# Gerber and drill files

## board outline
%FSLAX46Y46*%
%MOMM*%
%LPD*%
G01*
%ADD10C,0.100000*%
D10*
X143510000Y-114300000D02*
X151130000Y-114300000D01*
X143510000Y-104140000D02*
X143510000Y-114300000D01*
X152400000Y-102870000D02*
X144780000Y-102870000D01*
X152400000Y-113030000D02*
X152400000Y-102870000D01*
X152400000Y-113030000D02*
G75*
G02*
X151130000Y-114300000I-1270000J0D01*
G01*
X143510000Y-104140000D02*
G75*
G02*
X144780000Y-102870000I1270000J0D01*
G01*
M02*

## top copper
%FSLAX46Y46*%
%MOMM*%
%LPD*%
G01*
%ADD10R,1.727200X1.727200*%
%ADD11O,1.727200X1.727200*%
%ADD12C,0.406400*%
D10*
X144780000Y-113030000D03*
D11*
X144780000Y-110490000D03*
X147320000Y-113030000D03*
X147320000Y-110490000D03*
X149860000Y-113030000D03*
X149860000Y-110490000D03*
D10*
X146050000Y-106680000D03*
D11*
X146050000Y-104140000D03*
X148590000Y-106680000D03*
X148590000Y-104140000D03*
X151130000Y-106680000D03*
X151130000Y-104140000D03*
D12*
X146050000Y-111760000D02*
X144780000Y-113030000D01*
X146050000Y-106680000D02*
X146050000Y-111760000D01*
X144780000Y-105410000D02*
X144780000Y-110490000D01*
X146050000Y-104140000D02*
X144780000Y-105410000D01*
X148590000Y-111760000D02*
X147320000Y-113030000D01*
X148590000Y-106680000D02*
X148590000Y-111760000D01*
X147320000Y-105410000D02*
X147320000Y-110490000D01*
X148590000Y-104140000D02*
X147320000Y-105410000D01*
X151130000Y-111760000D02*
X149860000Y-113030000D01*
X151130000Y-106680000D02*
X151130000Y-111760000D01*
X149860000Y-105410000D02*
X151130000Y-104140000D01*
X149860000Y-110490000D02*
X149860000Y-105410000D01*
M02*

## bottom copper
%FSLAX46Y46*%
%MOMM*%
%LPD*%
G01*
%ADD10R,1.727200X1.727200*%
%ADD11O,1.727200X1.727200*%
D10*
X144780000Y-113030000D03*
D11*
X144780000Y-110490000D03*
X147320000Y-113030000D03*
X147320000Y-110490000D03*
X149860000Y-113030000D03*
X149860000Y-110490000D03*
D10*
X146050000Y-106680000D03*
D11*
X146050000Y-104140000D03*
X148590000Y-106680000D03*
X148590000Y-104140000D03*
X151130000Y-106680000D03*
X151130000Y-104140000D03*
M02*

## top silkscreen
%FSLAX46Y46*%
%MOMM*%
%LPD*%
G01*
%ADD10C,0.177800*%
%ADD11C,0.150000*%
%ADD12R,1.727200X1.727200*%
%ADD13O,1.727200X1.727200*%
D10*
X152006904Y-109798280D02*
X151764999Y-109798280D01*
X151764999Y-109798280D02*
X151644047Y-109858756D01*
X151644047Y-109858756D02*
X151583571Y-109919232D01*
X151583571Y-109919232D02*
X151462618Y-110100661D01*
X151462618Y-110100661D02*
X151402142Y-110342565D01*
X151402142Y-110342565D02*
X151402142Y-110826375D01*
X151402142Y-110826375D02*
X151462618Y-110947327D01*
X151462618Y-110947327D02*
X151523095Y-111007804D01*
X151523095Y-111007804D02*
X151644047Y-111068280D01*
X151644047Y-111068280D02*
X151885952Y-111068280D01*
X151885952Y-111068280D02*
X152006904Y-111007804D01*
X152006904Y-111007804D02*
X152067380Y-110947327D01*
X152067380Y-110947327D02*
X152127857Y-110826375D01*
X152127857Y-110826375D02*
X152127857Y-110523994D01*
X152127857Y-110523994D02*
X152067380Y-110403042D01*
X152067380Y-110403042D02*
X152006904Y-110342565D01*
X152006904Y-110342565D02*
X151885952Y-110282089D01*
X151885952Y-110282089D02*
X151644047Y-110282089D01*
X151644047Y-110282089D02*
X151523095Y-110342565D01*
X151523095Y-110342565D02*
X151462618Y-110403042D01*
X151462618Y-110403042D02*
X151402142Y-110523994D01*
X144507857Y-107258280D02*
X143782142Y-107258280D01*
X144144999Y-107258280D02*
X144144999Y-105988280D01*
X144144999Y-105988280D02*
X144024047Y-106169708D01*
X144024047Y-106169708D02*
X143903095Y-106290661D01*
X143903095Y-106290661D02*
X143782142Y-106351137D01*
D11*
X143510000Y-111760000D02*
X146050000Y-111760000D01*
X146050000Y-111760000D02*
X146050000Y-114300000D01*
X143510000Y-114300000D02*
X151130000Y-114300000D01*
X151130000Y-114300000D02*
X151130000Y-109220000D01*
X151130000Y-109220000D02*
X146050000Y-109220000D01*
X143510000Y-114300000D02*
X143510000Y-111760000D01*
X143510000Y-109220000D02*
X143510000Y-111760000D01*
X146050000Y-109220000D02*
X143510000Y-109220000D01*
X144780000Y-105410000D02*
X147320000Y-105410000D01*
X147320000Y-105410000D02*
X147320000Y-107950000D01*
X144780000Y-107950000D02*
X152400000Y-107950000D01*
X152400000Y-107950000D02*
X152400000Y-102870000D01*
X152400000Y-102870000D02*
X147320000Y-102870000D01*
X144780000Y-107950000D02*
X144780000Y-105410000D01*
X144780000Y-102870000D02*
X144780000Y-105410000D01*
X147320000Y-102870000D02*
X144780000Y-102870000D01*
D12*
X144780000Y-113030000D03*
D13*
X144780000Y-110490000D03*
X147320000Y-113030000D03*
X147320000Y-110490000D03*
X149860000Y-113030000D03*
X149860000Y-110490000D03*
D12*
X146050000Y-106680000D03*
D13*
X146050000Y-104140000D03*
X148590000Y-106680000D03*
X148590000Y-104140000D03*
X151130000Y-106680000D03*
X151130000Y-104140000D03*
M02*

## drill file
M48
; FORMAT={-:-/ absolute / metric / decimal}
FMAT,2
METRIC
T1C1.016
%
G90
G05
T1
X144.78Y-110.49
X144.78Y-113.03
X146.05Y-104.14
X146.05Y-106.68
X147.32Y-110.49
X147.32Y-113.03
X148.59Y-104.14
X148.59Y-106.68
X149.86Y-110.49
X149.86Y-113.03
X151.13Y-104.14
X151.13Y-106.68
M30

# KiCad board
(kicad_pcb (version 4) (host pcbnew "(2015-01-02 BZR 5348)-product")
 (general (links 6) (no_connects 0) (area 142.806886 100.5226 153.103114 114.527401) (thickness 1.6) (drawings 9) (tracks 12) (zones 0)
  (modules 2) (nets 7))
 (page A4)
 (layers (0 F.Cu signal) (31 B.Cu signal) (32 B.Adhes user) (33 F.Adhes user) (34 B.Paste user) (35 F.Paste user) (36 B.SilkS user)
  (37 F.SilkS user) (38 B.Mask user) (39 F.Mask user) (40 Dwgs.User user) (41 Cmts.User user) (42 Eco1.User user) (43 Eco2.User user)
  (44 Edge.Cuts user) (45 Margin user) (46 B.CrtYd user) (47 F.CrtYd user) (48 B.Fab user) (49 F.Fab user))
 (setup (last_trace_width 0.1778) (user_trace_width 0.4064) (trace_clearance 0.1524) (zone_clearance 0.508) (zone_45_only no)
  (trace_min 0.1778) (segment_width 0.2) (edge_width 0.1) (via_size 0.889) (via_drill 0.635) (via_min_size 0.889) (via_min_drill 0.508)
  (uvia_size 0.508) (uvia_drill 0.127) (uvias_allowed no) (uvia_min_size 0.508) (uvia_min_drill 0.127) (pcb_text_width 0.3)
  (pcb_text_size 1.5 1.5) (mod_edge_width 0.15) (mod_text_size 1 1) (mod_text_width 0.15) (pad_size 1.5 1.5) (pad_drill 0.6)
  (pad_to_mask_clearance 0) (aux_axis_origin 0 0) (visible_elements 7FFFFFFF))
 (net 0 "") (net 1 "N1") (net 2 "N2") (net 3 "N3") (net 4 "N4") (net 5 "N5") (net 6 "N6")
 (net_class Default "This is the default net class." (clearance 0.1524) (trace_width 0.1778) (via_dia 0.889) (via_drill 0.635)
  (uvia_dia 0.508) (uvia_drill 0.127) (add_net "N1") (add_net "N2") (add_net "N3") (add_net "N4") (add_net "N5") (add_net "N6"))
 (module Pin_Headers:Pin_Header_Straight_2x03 (layer F.Cu) (at 147.32 111.76)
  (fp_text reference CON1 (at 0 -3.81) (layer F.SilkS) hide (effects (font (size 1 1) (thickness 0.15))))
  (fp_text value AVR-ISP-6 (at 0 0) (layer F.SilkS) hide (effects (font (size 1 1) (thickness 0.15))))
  (fp_line (start -3.81 0) (end -1.27 0) (layer F.SilkS) (width 0.15))
  (fp_line (start -1.27 0) (end -1.27 2.54) (layer F.SilkS) (width 0.15))
  (fp_line (start -3.81 2.54) (end 3.81 2.54) (layer F.SilkS) (width 0.15))
  (fp_line (start 3.81 2.54) (end 3.81 -2.54) (layer F.SilkS) (width 0.15))
  (fp_line (start 3.81 -2.54) (end -1.27 -2.54) (layer F.SilkS) (width 0.15))
  (fp_line (start -3.81 2.54) (end -3.81 0) (layer F.SilkS) (width 0.15))
  (fp_line (start -3.81 -2.54) (end -3.81 0) (layer F.SilkS) (width 0.15))
  (fp_line (start -1.27 -2.54) (end -3.81 -2.54) (layer F.SilkS) (width 0.15))
  (pad 1 thru_hole rect (at -2.54 1.27) (size 1.7272 1.7272) (drill 1.016) (layers *.Cu *.Mask F.SilkS) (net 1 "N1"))
  (pad 2 thru_hole oval (at -2.54 -1.27) (size 1.7272 1.7272) (drill 1.016) (layers *.Cu *.Mask F.SilkS) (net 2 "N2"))
  (pad 3 thru_hole oval (at 0 1.27) (size 1.7272 1.7272) (drill 1.016) (layers *.Cu *.Mask F.SilkS) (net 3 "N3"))
  (pad 4 thru_hole oval (at 0 -1.27) (size 1.7272 1.7272) (drill 1.016) (layers *.Cu *.Mask F.SilkS) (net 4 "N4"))
  (pad 5 thru_hole oval (at 2.54 1.27) (size 1.7272 1.7272) (drill 1.016) (layers *.Cu *.Mask F.SilkS) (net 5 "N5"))
  (pad 6 thru_hole oval (at 2.54 -1.27) (size 1.7272 1.7272) (drill 1.016) (layers *.Cu *.Mask F.SilkS) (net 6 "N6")))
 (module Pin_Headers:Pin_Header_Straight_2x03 (layer F.Cu) (at 148.59 105.41)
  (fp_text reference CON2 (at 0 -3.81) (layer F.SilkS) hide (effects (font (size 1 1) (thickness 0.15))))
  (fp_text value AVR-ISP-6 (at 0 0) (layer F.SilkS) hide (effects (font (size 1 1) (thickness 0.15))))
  (fp_line (start -3.81 0) (end -1.27 0) (layer F.SilkS) (width 0.15))
  (fp_line (start -1.27 0) (end -1.27 2.54) (layer F.SilkS) (width 0.15))
  (fp_line (start -3.81 2.54) (end 3.81 2.54) (layer F.SilkS) (width 0.15))
  (fp_line (start 3.81 2.54) (end 3.81 -2.54) (layer F.SilkS) (width 0.15))
  (fp_line (start 3.81 -2.54) (end -1.27 -2.54) (layer F.SilkS) (width 0.15))
  (fp_line (start -3.81 2.54) (end -3.81 0) (layer F.SilkS) (width 0.15))
  (fp_line (start -3.81 -2.54) (end -3.81 0) (layer F.SilkS) (width 0.15))
  (fp_line (start -1.27 -2.54) (end -3.81 -2.54) (layer F.SilkS) (width 0.15))
  (pad 1 thru_hole rect (at -2.54 1.27) (size 1.7272 1.7272) (drill 1.016) (layers *.Cu *.Mask F.SilkS) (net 1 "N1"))
  (pad 2 thru_hole oval (at -2.54 -1.27) (size 1.7272 1.7272) (drill 1.016) (layers *.Cu *.Mask F.SilkS) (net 2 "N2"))
  (pad 3 thru_hole oval (at 0 1.27) (size 1.7272 1.7272) (drill 1.016) (layers *.Cu *.Mask F.SilkS) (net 3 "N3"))
  (pad 4 thru_hole oval (at 0 -1.27) (size 1.7272 1.7272) (drill 1.016) (layers *.Cu *.Mask F.SilkS) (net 4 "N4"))
  (pad 5 thru_hole oval (at 2.54 1.27) (size 1.7272 1.7272) (drill 1.016) (layers *.Cu *.Mask F.SilkS) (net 5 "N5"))
  (pad 6 thru_hole oval (at 2.54 -1.27) (size 1.7272 1.7272) (drill 1.016) (layers *.Cu *.Mask F.SilkS) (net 6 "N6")))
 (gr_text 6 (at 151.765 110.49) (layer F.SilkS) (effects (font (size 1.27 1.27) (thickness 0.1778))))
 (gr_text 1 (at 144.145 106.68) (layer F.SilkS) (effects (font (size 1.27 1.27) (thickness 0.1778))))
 (gr_line (start 143.51 114.3) (end 151.13 114.3) (angle 90) (layer Edge.Cuts) (width 0.1))
 (gr_line (start 143.51 104.14) (end 143.51 114.3) (angle 90) (layer Edge.Cuts) (width 0.1))
 (gr_line (start 152.4 102.87) (end 144.78 102.87) (angle 90) (layer Edge.Cuts) (width 0.1))
 (gr_line (start 152.4 113.03) (end 152.4 102.87) (angle 90) (layer Edge.Cuts) (width 0.1))
 (gr_arc (start 151.13 113.03) (end 152.4 113.03) (angle 90) (layer Edge.Cuts) (width 0.1))
 (gr_arc (start 144.78 104.14) (end 143.51 104.14) (angle 90) (layer Edge.Cuts) (width 0.1))
 (segment (start 146.05 111.76) (end 144.78 113.03) (width 0.4064) (layer F.Cu) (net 1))
 (segment (start 146.05 106.68) (end 146.05 111.76) (width 0.4064) (layer F.Cu) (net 1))
 (segment (start 144.78 105.41) (end 144.78 110.49) (width 0.4064) (layer F.Cu) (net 2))
 (segment (start 146.05 104.14) (end 144.78 105.41) (width 0.4064) (layer F.Cu) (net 2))
 (segment (start 148.59 111.76) (end 147.32 113.03) (width 0.4064) (layer F.Cu) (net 3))
 (segment (start 148.59 106.68) (end 148.59 111.76) (width 0.4064) (layer F.Cu) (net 3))
 (segment (start 147.32 105.41) (end 147.32 110.49) (width 0.4064) (layer F.Cu) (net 4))
 (segment (start 148.59 104.14) (end 147.32 105.41) (width 0.4064) (layer F.Cu) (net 4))
 (segment (start 151.13 111.76) (end 149.86 113.03) (width 0.4064) (layer F.Cu) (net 5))
 (segment (start 151.13 106.68) (end 151.13 111.76) (width 0.4064) (layer F.Cu) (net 5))
 (segment (start 149.86 105.41) (end 151.13 104.14) (width 0.4064) (layer F.Cu) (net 6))
 (segment (start 149.86 110.49) (end 149.86 105.41) (width 0.4064) (layer F.Cu) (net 6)))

